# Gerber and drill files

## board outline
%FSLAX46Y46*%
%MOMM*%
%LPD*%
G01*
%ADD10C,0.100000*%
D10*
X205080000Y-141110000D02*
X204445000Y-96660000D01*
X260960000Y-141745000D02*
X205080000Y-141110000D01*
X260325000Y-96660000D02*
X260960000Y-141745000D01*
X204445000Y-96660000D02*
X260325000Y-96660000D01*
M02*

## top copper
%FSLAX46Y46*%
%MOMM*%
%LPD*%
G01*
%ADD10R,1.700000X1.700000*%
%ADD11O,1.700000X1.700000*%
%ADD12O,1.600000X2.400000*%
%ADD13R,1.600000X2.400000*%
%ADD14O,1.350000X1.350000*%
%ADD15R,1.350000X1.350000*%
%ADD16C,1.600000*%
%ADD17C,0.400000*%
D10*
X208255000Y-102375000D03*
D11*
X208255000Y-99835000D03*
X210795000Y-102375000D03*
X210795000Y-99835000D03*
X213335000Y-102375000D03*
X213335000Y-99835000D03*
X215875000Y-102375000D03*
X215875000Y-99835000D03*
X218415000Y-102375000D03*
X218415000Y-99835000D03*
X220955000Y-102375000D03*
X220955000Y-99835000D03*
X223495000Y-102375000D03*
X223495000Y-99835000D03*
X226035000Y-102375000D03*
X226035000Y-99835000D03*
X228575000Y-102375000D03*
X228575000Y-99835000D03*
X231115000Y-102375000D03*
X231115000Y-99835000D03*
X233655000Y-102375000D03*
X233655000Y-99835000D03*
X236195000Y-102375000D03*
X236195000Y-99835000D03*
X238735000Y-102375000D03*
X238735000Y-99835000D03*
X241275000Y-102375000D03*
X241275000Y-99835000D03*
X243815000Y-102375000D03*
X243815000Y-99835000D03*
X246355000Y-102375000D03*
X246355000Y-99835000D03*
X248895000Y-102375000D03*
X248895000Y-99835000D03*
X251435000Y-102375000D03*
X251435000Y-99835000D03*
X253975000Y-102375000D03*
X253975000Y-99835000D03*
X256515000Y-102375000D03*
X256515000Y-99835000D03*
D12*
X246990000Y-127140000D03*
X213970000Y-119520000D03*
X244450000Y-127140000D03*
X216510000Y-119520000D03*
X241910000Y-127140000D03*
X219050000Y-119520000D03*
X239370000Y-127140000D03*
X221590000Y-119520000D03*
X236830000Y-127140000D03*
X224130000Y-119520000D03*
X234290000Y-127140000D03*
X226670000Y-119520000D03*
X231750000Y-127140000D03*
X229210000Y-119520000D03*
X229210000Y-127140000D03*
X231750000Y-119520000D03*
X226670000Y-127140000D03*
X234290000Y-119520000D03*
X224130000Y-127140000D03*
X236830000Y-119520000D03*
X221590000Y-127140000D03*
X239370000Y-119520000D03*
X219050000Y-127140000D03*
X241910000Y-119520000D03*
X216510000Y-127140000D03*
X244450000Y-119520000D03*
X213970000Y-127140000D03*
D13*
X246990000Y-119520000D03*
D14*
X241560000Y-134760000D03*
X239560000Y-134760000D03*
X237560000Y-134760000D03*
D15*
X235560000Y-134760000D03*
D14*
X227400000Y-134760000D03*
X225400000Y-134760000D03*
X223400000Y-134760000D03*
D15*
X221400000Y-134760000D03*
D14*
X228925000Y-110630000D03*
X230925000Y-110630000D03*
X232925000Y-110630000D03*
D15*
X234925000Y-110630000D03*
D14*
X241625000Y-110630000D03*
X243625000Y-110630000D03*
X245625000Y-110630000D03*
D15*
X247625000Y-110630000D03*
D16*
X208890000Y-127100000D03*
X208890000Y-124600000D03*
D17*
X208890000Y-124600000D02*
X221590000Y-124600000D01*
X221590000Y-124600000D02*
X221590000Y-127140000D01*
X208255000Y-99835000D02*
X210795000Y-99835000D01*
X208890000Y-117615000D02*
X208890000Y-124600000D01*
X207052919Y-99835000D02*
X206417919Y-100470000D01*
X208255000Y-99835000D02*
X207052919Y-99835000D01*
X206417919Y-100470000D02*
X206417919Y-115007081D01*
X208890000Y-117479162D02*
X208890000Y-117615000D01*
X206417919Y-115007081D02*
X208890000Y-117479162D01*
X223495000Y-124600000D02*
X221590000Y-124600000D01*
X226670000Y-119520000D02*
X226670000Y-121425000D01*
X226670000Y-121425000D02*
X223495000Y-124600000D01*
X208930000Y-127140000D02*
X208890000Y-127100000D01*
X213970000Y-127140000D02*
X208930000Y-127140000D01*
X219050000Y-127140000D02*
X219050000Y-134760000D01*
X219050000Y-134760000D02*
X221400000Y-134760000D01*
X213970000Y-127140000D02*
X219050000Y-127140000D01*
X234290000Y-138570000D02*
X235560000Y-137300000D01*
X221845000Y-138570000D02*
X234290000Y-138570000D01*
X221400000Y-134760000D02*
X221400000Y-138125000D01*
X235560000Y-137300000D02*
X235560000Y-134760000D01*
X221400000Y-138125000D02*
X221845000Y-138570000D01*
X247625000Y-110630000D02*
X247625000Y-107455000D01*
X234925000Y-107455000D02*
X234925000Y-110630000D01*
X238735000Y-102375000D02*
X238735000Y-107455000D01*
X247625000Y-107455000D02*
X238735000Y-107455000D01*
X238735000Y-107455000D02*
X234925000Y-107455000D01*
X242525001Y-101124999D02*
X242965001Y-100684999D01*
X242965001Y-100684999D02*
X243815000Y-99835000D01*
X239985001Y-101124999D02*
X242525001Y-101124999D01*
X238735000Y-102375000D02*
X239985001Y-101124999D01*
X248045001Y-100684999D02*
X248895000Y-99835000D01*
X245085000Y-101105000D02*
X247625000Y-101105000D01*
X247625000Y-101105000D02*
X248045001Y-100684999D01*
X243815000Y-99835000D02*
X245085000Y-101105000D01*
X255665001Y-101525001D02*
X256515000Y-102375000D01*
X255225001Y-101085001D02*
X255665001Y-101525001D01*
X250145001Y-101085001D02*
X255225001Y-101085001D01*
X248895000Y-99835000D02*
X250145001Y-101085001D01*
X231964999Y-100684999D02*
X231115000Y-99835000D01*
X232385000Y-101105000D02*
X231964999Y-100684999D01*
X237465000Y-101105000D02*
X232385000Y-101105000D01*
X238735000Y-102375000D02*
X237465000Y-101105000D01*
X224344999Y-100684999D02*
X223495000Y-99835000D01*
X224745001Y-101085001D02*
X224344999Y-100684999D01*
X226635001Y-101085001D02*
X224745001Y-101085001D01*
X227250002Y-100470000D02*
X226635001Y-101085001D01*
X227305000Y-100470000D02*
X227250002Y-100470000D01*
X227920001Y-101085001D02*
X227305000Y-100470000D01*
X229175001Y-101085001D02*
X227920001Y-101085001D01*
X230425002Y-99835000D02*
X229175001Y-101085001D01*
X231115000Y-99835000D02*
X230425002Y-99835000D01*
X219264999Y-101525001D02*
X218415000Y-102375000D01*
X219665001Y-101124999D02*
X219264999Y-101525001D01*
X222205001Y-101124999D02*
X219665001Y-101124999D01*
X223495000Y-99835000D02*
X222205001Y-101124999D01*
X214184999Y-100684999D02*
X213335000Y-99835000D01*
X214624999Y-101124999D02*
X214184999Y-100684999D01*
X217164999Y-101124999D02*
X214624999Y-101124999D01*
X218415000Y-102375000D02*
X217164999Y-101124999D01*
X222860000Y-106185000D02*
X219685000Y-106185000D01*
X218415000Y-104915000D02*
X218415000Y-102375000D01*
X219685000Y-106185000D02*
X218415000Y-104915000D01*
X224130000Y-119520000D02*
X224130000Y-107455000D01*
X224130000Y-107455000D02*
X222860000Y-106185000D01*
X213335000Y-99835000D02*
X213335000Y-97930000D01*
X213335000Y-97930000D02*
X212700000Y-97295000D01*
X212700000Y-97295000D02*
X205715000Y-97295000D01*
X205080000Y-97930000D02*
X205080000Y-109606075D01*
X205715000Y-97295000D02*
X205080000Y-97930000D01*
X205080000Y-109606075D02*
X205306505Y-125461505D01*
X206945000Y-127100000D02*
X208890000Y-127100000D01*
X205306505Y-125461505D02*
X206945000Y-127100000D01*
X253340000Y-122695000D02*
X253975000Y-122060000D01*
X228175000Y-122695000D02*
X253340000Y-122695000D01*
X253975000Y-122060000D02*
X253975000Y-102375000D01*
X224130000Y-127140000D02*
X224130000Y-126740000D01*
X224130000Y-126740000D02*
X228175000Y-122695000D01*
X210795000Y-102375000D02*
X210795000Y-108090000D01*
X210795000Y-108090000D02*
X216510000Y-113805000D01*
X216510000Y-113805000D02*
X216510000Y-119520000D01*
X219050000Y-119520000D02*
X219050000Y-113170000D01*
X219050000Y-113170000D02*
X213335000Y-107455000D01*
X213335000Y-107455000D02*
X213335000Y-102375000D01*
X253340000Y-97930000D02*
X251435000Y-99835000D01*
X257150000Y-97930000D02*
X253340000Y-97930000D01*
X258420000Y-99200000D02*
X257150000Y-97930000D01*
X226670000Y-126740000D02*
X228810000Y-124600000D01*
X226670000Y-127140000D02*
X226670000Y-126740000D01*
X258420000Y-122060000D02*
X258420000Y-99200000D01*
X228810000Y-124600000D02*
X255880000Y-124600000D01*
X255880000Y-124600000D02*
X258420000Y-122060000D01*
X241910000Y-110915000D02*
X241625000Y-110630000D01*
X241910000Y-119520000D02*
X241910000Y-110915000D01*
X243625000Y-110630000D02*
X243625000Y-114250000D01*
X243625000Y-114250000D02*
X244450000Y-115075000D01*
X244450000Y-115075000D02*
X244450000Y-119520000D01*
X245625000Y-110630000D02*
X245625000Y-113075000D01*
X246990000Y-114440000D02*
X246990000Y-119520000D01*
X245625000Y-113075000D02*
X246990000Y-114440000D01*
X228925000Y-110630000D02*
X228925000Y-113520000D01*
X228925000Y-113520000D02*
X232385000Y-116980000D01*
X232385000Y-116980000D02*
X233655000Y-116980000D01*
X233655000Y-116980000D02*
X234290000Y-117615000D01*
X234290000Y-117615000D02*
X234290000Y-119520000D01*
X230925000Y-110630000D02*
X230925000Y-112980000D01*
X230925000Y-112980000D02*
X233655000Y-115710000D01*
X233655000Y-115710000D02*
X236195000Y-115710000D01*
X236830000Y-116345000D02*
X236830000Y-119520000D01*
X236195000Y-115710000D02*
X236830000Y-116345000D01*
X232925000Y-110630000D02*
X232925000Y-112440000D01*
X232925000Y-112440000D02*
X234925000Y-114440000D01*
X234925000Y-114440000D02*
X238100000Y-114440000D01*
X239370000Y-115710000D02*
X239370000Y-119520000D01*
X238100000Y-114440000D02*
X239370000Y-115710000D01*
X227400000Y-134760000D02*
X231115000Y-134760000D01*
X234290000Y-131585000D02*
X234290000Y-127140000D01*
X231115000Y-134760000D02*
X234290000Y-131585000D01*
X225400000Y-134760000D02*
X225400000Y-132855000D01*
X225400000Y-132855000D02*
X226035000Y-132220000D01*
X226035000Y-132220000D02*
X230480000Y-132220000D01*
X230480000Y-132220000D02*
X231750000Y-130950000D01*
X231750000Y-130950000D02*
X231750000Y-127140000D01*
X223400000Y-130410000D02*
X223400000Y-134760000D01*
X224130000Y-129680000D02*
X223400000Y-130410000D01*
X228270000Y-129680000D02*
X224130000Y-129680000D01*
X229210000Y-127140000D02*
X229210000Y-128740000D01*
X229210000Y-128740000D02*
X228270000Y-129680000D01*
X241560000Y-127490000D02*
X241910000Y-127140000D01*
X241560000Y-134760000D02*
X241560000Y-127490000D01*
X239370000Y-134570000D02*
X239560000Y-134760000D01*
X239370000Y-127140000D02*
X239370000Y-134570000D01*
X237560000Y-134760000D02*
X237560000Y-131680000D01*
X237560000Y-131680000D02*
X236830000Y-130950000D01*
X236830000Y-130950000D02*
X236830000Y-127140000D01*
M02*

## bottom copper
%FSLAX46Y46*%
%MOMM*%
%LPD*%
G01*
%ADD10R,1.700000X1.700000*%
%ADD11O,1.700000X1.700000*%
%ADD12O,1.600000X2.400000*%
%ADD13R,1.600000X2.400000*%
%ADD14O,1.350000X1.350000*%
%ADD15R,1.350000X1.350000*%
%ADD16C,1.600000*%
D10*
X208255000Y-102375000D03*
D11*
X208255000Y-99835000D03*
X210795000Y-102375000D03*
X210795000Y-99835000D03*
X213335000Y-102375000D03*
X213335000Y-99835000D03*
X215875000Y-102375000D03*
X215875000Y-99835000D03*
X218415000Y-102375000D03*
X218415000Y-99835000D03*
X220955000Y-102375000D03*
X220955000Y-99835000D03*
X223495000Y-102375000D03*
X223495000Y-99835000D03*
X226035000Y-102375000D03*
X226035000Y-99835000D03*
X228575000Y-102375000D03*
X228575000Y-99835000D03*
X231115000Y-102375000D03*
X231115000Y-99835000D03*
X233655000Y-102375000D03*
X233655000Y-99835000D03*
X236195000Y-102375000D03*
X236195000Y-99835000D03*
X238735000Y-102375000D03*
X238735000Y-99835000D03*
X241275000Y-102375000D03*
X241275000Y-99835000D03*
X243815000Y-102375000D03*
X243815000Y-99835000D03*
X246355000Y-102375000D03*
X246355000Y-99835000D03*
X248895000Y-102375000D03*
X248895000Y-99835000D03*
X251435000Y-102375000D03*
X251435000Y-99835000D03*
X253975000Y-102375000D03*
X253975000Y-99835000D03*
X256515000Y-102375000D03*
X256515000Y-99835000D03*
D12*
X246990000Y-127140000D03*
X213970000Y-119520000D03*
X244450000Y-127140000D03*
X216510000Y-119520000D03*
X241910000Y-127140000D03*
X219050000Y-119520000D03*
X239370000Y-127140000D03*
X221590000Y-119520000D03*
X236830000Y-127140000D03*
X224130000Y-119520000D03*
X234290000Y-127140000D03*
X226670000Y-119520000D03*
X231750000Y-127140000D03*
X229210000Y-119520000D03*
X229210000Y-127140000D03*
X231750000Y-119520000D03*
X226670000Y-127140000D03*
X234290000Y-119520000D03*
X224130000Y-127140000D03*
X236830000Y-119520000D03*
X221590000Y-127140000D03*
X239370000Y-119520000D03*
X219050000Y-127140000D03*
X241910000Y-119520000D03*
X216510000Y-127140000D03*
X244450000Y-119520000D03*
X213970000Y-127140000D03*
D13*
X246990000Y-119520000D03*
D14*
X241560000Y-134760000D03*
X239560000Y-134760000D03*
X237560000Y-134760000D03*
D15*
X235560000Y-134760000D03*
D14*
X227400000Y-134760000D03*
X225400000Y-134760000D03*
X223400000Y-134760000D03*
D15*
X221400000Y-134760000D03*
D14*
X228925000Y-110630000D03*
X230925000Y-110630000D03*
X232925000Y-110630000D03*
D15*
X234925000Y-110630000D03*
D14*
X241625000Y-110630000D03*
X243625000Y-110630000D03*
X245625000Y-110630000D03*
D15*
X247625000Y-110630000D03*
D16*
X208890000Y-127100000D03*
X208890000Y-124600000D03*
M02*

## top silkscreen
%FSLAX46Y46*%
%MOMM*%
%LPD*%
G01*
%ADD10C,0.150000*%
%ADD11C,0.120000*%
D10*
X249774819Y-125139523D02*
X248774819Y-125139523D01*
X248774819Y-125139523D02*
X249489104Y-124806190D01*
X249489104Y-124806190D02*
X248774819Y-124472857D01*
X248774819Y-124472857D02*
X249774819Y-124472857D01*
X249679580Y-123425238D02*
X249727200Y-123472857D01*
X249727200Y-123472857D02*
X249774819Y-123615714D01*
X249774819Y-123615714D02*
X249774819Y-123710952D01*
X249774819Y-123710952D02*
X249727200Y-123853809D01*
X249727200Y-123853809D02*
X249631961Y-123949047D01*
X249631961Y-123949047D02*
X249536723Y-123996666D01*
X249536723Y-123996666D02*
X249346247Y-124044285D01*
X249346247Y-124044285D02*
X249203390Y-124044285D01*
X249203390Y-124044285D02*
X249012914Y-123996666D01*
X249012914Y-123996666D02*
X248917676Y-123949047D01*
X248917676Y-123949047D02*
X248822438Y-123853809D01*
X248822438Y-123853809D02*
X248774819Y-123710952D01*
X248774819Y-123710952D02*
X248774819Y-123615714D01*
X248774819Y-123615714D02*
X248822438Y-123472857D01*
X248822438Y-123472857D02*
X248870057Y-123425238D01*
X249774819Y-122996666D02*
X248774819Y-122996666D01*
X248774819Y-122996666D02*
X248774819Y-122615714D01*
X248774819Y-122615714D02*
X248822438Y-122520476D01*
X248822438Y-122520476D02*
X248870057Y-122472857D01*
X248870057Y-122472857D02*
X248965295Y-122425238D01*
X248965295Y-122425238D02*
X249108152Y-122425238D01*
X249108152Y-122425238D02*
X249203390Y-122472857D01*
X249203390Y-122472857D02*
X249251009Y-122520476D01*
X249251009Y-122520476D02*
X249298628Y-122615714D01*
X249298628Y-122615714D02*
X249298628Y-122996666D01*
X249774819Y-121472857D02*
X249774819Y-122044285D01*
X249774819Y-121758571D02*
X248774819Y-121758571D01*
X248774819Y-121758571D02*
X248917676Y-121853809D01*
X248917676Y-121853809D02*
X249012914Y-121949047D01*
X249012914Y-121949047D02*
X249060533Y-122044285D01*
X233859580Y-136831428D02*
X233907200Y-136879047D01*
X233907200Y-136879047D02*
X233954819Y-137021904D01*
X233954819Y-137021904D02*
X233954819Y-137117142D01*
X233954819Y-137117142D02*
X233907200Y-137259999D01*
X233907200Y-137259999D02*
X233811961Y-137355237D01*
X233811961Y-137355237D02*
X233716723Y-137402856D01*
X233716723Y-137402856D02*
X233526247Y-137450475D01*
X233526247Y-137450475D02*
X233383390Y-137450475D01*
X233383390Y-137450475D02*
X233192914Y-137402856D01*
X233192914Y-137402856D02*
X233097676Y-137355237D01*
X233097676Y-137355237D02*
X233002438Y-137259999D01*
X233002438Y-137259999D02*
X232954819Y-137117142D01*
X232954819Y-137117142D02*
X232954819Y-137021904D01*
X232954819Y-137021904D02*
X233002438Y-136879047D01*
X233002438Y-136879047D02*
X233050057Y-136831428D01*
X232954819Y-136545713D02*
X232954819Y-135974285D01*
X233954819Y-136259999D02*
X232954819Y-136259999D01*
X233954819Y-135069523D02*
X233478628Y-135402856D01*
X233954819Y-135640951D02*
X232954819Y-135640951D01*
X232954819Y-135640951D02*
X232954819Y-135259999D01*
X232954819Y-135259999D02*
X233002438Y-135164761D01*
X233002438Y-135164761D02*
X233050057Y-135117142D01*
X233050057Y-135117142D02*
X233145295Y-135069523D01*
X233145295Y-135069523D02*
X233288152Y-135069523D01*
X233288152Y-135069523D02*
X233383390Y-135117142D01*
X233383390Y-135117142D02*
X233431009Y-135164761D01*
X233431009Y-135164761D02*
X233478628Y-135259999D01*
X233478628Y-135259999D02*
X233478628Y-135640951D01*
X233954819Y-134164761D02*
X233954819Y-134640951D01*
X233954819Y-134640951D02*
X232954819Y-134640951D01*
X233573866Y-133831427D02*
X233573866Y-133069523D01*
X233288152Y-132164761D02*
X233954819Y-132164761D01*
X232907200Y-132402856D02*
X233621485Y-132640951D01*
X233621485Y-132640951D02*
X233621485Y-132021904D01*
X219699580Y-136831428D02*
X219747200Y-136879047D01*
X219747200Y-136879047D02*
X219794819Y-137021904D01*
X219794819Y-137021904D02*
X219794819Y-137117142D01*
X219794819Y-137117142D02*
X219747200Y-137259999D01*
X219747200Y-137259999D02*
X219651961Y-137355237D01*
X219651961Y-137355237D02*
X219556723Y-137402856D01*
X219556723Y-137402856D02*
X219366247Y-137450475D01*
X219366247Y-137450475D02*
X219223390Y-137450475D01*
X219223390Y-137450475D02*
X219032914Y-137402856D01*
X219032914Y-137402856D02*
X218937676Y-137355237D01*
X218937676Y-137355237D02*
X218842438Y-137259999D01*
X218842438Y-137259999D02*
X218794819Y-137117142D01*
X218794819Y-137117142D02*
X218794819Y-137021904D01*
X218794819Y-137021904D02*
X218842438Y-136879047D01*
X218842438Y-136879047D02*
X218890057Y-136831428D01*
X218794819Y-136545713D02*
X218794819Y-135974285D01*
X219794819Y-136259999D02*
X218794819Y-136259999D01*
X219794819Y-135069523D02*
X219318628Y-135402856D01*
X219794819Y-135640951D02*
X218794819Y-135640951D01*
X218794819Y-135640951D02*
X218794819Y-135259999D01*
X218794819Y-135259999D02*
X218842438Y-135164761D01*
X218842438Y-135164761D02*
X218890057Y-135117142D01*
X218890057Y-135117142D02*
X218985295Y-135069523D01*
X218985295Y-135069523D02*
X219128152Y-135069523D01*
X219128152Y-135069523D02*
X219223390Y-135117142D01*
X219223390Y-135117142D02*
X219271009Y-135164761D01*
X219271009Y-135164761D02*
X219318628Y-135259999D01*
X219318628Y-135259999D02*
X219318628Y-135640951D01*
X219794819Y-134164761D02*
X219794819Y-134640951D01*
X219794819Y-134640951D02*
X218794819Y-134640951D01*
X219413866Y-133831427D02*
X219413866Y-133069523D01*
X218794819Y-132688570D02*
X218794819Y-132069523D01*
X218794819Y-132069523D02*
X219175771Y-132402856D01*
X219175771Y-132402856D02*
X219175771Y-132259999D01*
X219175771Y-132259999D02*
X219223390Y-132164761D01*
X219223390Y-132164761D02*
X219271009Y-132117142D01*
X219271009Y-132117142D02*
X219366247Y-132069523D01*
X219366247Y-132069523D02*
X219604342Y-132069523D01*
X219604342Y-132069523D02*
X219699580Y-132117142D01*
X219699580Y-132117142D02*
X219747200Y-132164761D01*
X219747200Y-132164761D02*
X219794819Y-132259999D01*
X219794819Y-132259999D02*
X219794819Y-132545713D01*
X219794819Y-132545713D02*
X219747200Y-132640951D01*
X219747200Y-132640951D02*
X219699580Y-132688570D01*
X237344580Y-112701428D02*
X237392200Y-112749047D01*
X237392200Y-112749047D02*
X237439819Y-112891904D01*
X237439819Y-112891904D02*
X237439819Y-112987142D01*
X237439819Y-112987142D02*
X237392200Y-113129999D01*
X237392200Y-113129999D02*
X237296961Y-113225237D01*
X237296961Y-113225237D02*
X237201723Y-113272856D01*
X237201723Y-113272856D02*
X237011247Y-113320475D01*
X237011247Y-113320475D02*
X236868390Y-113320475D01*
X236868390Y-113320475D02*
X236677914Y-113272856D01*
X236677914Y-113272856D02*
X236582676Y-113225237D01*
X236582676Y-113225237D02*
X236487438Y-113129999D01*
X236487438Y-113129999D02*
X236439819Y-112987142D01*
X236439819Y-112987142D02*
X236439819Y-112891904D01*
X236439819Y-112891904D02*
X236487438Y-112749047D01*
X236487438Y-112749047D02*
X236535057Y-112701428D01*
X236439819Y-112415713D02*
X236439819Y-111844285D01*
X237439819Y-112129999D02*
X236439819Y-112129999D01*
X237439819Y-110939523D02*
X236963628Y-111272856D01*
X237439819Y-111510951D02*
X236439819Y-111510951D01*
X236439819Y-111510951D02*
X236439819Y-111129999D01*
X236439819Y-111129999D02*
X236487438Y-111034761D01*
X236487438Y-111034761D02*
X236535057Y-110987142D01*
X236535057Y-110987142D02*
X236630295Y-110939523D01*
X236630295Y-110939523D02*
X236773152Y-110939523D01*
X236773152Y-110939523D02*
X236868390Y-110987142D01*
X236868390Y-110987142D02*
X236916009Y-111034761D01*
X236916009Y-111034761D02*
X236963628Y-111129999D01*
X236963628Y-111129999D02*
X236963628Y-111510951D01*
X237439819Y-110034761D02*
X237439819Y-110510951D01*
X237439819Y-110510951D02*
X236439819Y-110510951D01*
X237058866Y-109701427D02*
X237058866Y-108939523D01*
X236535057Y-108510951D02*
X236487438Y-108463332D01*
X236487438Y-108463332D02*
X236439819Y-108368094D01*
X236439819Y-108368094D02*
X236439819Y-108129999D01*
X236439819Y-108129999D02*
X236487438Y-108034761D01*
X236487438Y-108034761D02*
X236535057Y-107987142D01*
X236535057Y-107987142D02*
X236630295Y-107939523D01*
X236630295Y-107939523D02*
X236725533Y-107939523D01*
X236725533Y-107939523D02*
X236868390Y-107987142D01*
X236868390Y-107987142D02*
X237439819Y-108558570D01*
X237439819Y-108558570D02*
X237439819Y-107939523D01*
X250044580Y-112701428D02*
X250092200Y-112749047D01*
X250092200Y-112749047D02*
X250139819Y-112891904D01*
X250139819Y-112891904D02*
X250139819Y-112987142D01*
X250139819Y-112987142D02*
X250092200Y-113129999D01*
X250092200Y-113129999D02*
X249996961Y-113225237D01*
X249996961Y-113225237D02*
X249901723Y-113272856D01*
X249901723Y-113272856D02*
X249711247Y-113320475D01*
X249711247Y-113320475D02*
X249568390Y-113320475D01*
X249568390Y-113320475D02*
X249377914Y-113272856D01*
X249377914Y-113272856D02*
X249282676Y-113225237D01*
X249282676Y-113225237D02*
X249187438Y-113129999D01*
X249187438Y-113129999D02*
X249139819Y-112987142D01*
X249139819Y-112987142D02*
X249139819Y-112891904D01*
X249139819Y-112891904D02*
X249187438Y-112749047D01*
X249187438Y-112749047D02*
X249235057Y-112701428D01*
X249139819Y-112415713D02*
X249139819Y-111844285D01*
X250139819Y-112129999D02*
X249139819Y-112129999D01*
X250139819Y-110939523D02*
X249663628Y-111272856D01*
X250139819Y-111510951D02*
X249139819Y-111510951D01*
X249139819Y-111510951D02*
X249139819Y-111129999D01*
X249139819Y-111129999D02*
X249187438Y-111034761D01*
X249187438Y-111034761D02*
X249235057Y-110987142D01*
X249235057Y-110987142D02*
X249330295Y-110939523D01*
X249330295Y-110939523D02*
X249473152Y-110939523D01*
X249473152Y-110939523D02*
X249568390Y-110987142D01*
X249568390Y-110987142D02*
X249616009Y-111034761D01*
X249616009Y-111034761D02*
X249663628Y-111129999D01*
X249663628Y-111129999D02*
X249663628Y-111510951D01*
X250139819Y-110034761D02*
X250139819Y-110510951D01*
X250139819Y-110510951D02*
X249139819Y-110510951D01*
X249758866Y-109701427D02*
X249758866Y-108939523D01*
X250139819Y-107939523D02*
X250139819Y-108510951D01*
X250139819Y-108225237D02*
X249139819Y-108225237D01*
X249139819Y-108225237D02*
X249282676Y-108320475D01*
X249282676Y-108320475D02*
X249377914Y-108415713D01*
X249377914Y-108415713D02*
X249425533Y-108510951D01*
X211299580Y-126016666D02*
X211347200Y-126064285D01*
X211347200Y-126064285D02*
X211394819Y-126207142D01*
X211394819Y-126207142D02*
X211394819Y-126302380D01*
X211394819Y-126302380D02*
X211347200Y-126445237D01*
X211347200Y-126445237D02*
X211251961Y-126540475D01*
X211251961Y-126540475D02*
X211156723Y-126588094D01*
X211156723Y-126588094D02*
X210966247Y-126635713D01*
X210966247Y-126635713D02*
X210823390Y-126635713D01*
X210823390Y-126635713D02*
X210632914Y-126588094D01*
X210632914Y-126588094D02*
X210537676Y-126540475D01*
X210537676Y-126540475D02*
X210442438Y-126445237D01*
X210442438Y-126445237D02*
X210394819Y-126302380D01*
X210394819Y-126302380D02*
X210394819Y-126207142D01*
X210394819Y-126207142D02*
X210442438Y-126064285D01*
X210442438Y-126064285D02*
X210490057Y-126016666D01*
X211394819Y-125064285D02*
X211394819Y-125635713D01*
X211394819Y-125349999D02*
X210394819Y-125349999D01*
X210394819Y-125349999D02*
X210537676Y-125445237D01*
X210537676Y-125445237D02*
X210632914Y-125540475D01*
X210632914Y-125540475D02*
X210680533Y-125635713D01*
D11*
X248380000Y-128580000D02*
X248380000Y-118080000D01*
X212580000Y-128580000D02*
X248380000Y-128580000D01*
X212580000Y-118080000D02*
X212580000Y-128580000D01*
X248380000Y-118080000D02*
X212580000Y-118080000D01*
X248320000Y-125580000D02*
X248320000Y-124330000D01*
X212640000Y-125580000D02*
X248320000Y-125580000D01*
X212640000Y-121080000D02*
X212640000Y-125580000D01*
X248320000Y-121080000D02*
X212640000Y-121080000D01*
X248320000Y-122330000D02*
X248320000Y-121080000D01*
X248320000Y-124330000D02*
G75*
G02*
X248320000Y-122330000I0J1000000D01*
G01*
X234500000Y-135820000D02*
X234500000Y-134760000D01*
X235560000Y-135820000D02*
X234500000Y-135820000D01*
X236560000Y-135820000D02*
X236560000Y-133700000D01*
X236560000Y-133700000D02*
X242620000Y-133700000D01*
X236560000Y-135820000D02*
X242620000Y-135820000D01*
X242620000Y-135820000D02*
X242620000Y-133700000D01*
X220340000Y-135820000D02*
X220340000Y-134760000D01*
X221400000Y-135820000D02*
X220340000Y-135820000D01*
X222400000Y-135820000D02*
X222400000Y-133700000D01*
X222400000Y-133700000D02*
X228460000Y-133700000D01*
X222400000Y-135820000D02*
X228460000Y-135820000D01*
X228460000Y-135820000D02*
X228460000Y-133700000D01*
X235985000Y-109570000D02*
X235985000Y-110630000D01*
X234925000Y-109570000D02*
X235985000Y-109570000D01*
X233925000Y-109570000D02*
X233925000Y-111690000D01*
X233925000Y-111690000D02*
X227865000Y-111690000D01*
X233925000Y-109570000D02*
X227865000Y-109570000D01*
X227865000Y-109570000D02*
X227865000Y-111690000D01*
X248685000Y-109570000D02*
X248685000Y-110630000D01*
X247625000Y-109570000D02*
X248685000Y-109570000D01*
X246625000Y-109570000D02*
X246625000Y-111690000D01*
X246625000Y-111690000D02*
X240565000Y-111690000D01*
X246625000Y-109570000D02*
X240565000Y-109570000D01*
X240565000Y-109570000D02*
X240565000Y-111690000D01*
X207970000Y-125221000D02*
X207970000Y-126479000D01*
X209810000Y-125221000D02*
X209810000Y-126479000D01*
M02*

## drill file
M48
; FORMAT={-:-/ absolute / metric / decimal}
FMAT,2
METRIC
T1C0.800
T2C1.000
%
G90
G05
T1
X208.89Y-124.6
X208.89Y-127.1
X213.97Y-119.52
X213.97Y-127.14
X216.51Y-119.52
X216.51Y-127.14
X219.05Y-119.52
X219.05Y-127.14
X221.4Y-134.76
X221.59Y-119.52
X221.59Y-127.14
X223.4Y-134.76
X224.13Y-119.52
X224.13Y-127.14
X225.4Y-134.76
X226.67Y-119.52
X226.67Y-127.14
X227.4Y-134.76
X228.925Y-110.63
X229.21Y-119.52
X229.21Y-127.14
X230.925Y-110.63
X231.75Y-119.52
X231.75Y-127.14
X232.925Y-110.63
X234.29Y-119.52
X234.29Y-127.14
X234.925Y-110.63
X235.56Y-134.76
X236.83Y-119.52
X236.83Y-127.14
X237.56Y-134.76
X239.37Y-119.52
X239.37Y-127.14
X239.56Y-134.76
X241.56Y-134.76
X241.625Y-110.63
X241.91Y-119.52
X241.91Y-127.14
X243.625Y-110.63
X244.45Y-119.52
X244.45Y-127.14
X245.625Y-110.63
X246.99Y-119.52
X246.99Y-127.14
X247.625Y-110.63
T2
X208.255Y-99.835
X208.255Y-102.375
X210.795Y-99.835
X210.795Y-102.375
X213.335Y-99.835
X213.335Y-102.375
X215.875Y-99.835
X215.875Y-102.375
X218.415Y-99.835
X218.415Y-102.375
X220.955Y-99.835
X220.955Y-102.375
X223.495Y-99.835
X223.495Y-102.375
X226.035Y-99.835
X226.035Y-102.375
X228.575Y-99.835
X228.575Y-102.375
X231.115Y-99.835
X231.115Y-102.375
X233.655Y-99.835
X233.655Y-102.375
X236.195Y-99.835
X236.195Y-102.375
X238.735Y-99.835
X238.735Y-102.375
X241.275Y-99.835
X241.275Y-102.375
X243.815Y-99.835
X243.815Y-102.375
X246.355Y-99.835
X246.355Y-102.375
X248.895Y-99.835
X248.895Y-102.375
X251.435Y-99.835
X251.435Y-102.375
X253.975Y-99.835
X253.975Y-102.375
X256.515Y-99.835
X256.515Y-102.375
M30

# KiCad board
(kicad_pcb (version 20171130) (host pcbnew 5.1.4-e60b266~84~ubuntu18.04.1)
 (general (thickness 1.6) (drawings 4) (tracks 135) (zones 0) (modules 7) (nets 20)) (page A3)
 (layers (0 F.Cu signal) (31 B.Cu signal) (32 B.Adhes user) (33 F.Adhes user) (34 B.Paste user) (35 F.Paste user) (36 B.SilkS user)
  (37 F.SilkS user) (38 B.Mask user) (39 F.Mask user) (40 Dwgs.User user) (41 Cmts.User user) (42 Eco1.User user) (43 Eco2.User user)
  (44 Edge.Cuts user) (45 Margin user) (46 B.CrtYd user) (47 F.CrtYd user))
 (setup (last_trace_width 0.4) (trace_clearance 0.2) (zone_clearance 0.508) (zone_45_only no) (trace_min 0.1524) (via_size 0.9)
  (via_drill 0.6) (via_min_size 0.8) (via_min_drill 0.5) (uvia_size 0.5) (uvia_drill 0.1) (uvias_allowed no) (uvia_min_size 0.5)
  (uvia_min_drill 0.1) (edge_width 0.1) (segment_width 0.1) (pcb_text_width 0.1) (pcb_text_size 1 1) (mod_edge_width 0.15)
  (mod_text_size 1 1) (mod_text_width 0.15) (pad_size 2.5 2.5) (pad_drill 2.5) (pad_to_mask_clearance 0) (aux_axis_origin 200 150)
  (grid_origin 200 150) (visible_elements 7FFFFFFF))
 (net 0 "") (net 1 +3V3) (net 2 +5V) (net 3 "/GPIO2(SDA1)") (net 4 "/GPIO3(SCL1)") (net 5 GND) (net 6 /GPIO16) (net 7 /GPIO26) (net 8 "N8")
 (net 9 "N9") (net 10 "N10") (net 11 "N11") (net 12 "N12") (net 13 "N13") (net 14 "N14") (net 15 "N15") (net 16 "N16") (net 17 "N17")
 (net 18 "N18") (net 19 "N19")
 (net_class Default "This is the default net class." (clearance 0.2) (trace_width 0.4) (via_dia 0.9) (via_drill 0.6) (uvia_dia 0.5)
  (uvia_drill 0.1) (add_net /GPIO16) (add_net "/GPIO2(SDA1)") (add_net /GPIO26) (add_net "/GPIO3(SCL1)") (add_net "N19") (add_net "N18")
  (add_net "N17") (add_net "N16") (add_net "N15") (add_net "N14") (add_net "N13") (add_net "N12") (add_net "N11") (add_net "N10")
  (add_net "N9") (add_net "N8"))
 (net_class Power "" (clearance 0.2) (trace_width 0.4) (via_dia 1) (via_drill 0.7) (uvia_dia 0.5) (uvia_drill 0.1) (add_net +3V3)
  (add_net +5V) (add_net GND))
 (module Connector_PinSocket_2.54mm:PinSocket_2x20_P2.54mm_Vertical (layer B.Cu) (at 208.255 102.375 270)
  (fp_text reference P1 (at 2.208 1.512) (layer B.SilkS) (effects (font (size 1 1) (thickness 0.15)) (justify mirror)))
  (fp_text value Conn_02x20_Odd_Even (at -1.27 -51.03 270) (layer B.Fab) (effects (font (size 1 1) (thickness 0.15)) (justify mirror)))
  (pad 1 thru_hole rect (at 0 0 270) (size 1.7 1.7) (drill 1) (layers *.Cu *.Mask) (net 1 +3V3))
  (pad 2 thru_hole oval (at -2.54 0 270) (size 1.7 1.7) (drill 1) (layers *.Cu *.Mask) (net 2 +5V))
  (pad 3 thru_hole oval (at 0 -2.54 270) (size 1.7 1.7) (drill 1) (layers *.Cu *.Mask) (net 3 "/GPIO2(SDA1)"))
  (pad 4 thru_hole oval (at -2.54 -2.54 270) (size 1.7 1.7) (drill 1) (layers *.Cu *.Mask) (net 2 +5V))
  (pad 5 thru_hole oval (at 0 -5.08 270) (size 1.7 1.7) (drill 1) (layers *.Cu *.Mask) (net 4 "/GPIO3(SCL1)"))
  (pad 6 thru_hole oval (at -2.54 -5.08 270) (size 1.7 1.7) (drill 1) (layers *.Cu *.Mask) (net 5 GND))
  (pad 7 thru_hole oval (at 0 -7.62 270) (size 1.7 1.7) (drill 1) (layers *.Cu *.Mask))
  (pad 8 thru_hole oval (at -2.54 -7.62 270) (size 1.7 1.7) (drill 1) (layers *.Cu *.Mask))
  (pad 9 thru_hole oval (at 0 -10.16 270) (size 1.7 1.7) (drill 1) (layers *.Cu *.Mask) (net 5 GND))
  (pad 10 thru_hole oval (at -2.54 -10.16 270) (size 1.7 1.7) (drill 1) (layers *.Cu *.Mask))
  (pad 11 thru_hole oval (at 0 -12.7 270) (size 1.7 1.7) (drill 1) (layers *.Cu *.Mask))
  (pad 12 thru_hole oval (at -2.54 -12.7 270) (size 1.7 1.7) (drill 1) (layers *.Cu *.Mask))
  (pad 13 thru_hole oval (at 0 -15.24 270) (size 1.7 1.7) (drill 1) (layers *.Cu *.Mask))
  (pad 14 thru_hole oval (at -2.54 -15.24 270) (size 1.7 1.7) (drill 1) (layers *.Cu *.Mask) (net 5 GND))
  (pad 15 thru_hole oval (at 0 -17.78 270) (size 1.7 1.7) (drill 1) (layers *.Cu *.Mask))
  (pad 16 thru_hole oval (at -2.54 -17.78 270) (size 1.7 1.7) (drill 1) (layers *.Cu *.Mask))
  (pad 17 thru_hole oval (at 0 -20.32 270) (size 1.7 1.7) (drill 1) (layers *.Cu *.Mask) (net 1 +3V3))
  (pad 18 thru_hole oval (at -2.54 -20.32 270) (size 1.7 1.7) (drill 1) (layers *.Cu *.Mask))
  (pad 19 thru_hole oval (at 0 -22.86 270) (size 1.7 1.7) (drill 1) (layers *.Cu *.Mask))
  (pad 20 thru_hole oval (at -2.54 -22.86 270) (size 1.7 1.7) (drill 1) (layers *.Cu *.Mask) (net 5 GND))
  (pad 21 thru_hole oval (at 0 -25.4 270) (size 1.7 1.7) (drill 1) (layers *.Cu *.Mask))
  (pad 22 thru_hole oval (at -2.54 -25.4 270) (size 1.7 1.7) (drill 1) (layers *.Cu *.Mask))
  (pad 23 thru_hole oval (at 0 -27.94 270) (size 1.7 1.7) (drill 1) (layers *.Cu *.Mask))
  (pad 24 thru_hole oval (at -2.54 -27.94 270) (size 1.7 1.7) (drill 1) (layers *.Cu *.Mask))
  (pad 25 thru_hole oval (at 0 -30.48 270) (size 1.7 1.7) (drill 1) (layers *.Cu *.Mask) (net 5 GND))
  (pad 26 thru_hole oval (at -2.54 -30.48 270) (size 1.7 1.7) (drill 1) (layers *.Cu *.Mask))
  (pad 27 thru_hole oval (at 0 -33.02 270) (size 1.7 1.7) (drill 1) (layers *.Cu *.Mask))
  (pad 28 thru_hole oval (at -2.54 -33.02 270) (size 1.7 1.7) (drill 1) (layers *.Cu *.Mask))
  (pad 29 thru_hole oval (at 0 -35.56 270) (size 1.7 1.7) (drill 1) (layers *.Cu *.Mask))
  (pad 30 thru_hole oval (at -2.54 -35.56 270) (size 1.7 1.7) (drill 1) (layers *.Cu *.Mask) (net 5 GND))
  (pad 31 thru_hole oval (at 0 -38.1 270) (size 1.7 1.7) (drill 1) (layers *.Cu *.Mask))
  (pad 32 thru_hole oval (at -2.54 -38.1 270) (size 1.7 1.7) (drill 1) (layers *.Cu *.Mask))
  (pad 33 thru_hole oval (at 0 -40.64 270) (size 1.7 1.7) (drill 1) (layers *.Cu *.Mask))
  (pad 34 thru_hole oval (at -2.54 -40.64 270) (size 1.7 1.7) (drill 1) (layers *.Cu *.Mask) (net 5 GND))
  (pad 35 thru_hole oval (at 0 -43.18 270) (size 1.7 1.7) (drill 1) (layers *.Cu *.Mask))
  (pad 36 thru_hole oval (at -2.54 -43.18 270) (size 1.7 1.7) (drill 1) (layers *.Cu *.Mask) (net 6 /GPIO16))
  (pad 37 thru_hole oval (at 0 -45.72 270) (size 1.7 1.7) (drill 1) (layers *.Cu *.Mask) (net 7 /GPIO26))
  (pad 38 thru_hole oval (at -2.54 -45.72 270) (size 1.7 1.7) (drill 1) (layers *.Cu *.Mask))
  (pad 39 thru_hole oval (at 0 -48.26 270) (size 1.7 1.7) (drill 1) (layers *.Cu *.Mask) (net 5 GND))
  (pad 40 thru_hole oval (at -2.54 -48.26 270) (size 1.7 1.7) (drill 1) (layers *.Cu *.Mask)))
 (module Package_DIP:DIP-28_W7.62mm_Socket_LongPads (layer F.Cu) (at 246.99 119.52 270)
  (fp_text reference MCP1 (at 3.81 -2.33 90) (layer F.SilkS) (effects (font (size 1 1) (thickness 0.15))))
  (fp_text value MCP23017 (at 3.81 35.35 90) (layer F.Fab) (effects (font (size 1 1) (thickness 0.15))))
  (fp_line (start 9.06 -1.39) (end -1.44 -1.39) (layer F.SilkS) (width 0.12))
  (fp_line (start 9.06 34.41) (end 9.06 -1.39) (layer F.SilkS) (width 0.12))
  (fp_line (start -1.44 34.41) (end 9.06 34.41) (layer F.SilkS) (width 0.12))
  (fp_line (start -1.44 -1.39) (end -1.44 34.41) (layer F.SilkS) (width 0.12))
  (fp_line (start 6.06 -1.33) (end 4.81 -1.33) (layer F.SilkS) (width 0.12))
  (fp_line (start 6.06 34.35) (end 6.06 -1.33) (layer F.SilkS) (width 0.12))
  (fp_line (start 1.56 34.35) (end 6.06 34.35) (layer F.SilkS) (width 0.12))
  (fp_line (start 1.56 -1.33) (end 1.56 34.35) (layer F.SilkS) (width 0.12))
  (fp_line (start 2.81 -1.33) (end 1.56 -1.33) (layer F.SilkS) (width 0.12))
  (fp_arc (start 3.81 -1.33) (end 2.81 -1.33) (angle -180) (layer F.SilkS) (width 0.12))
  (pad 28 thru_hole oval (at 7.62 0 270) (size 2.4 1.6) (drill 0.8) (layers *.Cu *.Mask))
  (pad 14 thru_hole oval (at 0 33.02 270) (size 2.4 1.6) (drill 0.8) (layers *.Cu *.Mask))
  (pad 27 thru_hole oval (at 7.62 2.54 270) (size 2.4 1.6) (drill 0.8) (layers *.Cu *.Mask))
  (pad 13 thru_hole oval (at 0 30.48 270) (size 2.4 1.6) (drill 0.8) (layers *.Cu *.Mask) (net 3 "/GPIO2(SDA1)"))
  (pad 26 thru_hole oval (at 7.62 5.08 270) (size 2.4 1.6) (drill 0.8) (layers *.Cu *.Mask) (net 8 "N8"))
  (pad 12 thru_hole oval (at 0 27.94 270) (size 2.4 1.6) (drill 0.8) (layers *.Cu *.Mask) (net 4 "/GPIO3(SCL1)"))
  (pad 25 thru_hole oval (at 7.62 7.62 270) (size 2.4 1.6) (drill 0.8) (layers *.Cu *.Mask) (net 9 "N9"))
  (pad 11 thru_hole oval (at 0 25.4 270) (size 2.4 1.6) (drill 0.8) (layers *.Cu *.Mask))
  (pad 24 thru_hole oval (at 7.62 10.16 270) (size 2.4 1.6) (drill 0.8) (layers *.Cu *.Mask) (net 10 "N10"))
  (pad 10 thru_hole oval (at 0 22.86 270) (size 2.4 1.6) (drill 0.8) (layers *.Cu *.Mask) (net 5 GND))
  (pad 23 thru_hole oval (at 7.62 12.7 270) (size 2.4 1.6) (drill 0.8) (layers *.Cu *.Mask) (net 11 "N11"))
  (pad 9 thru_hole oval (at 0 20.32 270) (size 2.4 1.6) (drill 0.8) (layers *.Cu *.Mask) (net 2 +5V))
  (pad 22 thru_hole oval (at 7.62 15.24 270) (size 2.4 1.6) (drill 0.8) (layers *.Cu *.Mask) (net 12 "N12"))
  (pad 8 thru_hole oval (at 0 17.78 270) (size 2.4 1.6) (drill 0.8) (layers *.Cu *.Mask))
  (pad 21 thru_hole oval (at 7.62 17.78 270) (size 2.4 1.6) (drill 0.8) (layers *.Cu *.Mask) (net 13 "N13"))
  (pad 7 thru_hole oval (at 0 15.24 270) (size 2.4 1.6) (drill 0.8) (layers *.Cu *.Mask))
  (pad 20 thru_hole oval (at 7.62 20.32 270) (size 2.4 1.6) (drill 0.8) (layers *.Cu *.Mask) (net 6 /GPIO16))
  (pad 6 thru_hole oval (at 0 12.7 270) (size 2.4 1.6) (drill 0.8) (layers *.Cu *.Mask) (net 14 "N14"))
  (pad 19 thru_hole oval (at 7.62 22.86 270) (size 2.4 1.6) (drill 0.8) (layers *.Cu *.Mask) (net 7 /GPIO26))
  (pad 5 thru_hole oval (at 0 10.16 270) (size 2.4 1.6) (drill 0.8) (layers *.Cu *.Mask) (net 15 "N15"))
  (pad 18 thru_hole oval (at 7.62 25.4 270) (size 2.4 1.6) (drill 0.8) (layers *.Cu *.Mask) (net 2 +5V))
  (pad 4 thru_hole oval (at 0 7.62 270) (size 2.4 1.6) (drill 0.8) (layers *.Cu *.Mask) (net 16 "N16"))
  (pad 17 thru_hole oval (at 7.62 27.94 270) (size 2.4 1.6) (drill 0.8) (layers *.Cu *.Mask) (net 5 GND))
  (pad 3 thru_hole oval (at 0 5.08 270) (size 2.4 1.6) (drill 0.8) (layers *.Cu *.Mask) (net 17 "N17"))
  (pad 16 thru_hole oval (at 7.62 30.48 270) (size 2.4 1.6) (drill 0.8) (layers *.Cu *.Mask) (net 5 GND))
  (pad 2 thru_hole oval (at 0 2.54 270) (size 2.4 1.6) (drill 0.8) (layers *.Cu *.Mask) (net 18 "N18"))
  (pad 15 thru_hole oval (at 7.62 33.02 270) (size 2.4 1.6) (drill 0.8) (layers *.Cu *.Mask) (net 5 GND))
  (pad 1 thru_hole rect (at 0 0 270) (size 2.4 1.6) (drill 0.8) (layers *.Cu *.Mask) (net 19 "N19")))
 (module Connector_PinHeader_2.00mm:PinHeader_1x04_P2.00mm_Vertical (layer F.Cu) (at 235.56 134.76 90)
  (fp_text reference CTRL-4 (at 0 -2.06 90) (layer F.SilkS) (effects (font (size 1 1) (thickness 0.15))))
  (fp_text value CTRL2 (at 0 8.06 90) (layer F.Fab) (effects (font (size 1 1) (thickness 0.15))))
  (fp_line (start -1.06 -1.06) (end 0 -1.06) (layer F.SilkS) (width 0.12))
  (fp_line (start -1.06 0) (end -1.06 -1.06) (layer F.SilkS) (width 0.12))
  (fp_line (start -1.06 1) (end 1.06 1) (layer F.SilkS) (width 0.12))
  (fp_line (start 1.06 1) (end 1.06 7.06) (layer F.SilkS) (width 0.12))
  (fp_line (start -1.06 1) (end -1.06 7.06) (layer F.SilkS) (width 0.12))
  (fp_line (start -1.06 7.06) (end 1.06 7.06) (layer F.SilkS) (width 0.12))
  (pad 4 thru_hole oval (at 0 6 90) (size 1.35 1.35) (drill 0.8) (layers *.Cu *.Mask) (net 8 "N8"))
  (pad 3 thru_hole oval (at 0 4 90) (size 1.35 1.35) (drill 0.8) (layers *.Cu *.Mask) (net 9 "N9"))
  (pad 2 thru_hole oval (at 0 2 90) (size 1.35 1.35) (drill 0.8) (layers *.Cu *.Mask) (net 10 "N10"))
  (pad 1 thru_hole rect (at 0 0 90) (size 1.35 1.35) (drill 0.8) (layers *.Cu *.Mask) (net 5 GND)))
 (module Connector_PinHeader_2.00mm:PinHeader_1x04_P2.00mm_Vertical (layer F.Cu) (at 221.4 134.76 90)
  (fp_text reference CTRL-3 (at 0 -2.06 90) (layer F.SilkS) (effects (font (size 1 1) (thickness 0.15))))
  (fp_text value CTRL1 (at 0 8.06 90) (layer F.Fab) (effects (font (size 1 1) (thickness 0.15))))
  (fp_line (start -1.06 -1.06) (end 0 -1.06) (layer F.SilkS) (width 0.12))
  (fp_line (start -1.06 0) (end -1.06 -1.06) (layer F.SilkS) (width 0.12))
  (fp_line (start -1.06 1) (end 1.06 1) (layer F.SilkS) (width 0.12))
  (fp_line (start 1.06 1) (end 1.06 7.06) (layer F.SilkS) (width 0.12))
  (fp_line (start -1.06 1) (end -1.06 7.06) (layer F.SilkS) (width 0.12))
  (fp_line (start -1.06 7.06) (end 1.06 7.06) (layer F.SilkS) (width 0.12))
  (pad 4 thru_hole oval (at 0 6 90) (size 1.35 1.35) (drill 0.8) (layers *.Cu *.Mask) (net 11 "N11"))
  (pad 3 thru_hole oval (at 0 4 90) (size 1.35 1.35) (drill 0.8) (layers *.Cu *.Mask) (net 12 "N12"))
  (pad 2 thru_hole oval (at 0 2 90) (size 1.35 1.35) (drill 0.8) (layers *.Cu *.Mask) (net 13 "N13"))
  (pad 1 thru_hole rect (at 0 0 90) (size 1.35 1.35) (drill 0.8) (layers *.Cu *.Mask) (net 5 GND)))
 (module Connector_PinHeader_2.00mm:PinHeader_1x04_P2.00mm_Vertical (layer F.Cu) (at 234.925 110.63 270)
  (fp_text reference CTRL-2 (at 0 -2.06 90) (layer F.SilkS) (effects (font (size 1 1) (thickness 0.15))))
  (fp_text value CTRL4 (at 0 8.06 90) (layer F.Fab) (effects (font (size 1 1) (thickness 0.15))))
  (fp_line (start -1.06 -1.06) (end 0 -1.06) (layer F.SilkS) (width 0.12))
  (fp_line (start -1.06 0) (end -1.06 -1.06) (layer F.SilkS) (width 0.12))
  (fp_line (start -1.06 1) (end 1.06 1) (layer F.SilkS) (width 0.12))
  (fp_line (start 1.06 1) (end 1.06 7.06) (layer F.SilkS) (width 0.12))
  (fp_line (start -1.06 1) (end -1.06 7.06) (layer F.SilkS) (width 0.12))
  (fp_line (start -1.06 7.06) (end 1.06 7.06) (layer F.SilkS) (width 0.12))
  (pad 4 thru_hole oval (at 0 6 270) (size 1.35 1.35) (drill 0.8) (layers *.Cu *.Mask) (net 14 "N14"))
  (pad 3 thru_hole oval (at 0 4 270) (size 1.35 1.35) (drill 0.8) (layers *.Cu *.Mask) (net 15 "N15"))
  (pad 2 thru_hole oval (at 0 2 270) (size 1.35 1.35) (drill 0.8) (layers *.Cu *.Mask) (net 16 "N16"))
  (pad 1 thru_hole rect (at 0 0 270) (size 1.35 1.35) (drill 0.8) (layers *.Cu *.Mask) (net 5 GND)))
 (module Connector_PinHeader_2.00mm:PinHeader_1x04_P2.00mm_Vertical (layer F.Cu) (at 247.625 110.63 270)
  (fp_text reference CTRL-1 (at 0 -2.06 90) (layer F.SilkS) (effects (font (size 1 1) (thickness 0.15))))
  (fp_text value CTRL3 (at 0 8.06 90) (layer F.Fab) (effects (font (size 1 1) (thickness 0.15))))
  (fp_line (start -1.06 -1.06) (end 0 -1.06) (layer F.SilkS) (width 0.12))
  (fp_line (start -1.06 0) (end -1.06 -1.06) (layer F.SilkS) (width 0.12))
  (fp_line (start -1.06 1) (end 1.06 1) (layer F.SilkS) (width 0.12))
  (fp_line (start 1.06 1) (end 1.06 7.06) (layer F.SilkS) (width 0.12))
  (fp_line (start -1.06 1) (end -1.06 7.06) (layer F.SilkS) (width 0.12))
  (fp_line (start -1.06 7.06) (end 1.06 7.06) (layer F.SilkS) (width 0.12))
  (pad 4 thru_hole oval (at 0 6 270) (size 1.35 1.35) (drill 0.8) (layers *.Cu *.Mask) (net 17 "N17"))
  (pad 3 thru_hole oval (at 0 4 270) (size 1.35 1.35) (drill 0.8) (layers *.Cu *.Mask) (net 18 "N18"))
  (pad 2 thru_hole oval (at 0 2 270) (size 1.35 1.35) (drill 0.8) (layers *.Cu *.Mask) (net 19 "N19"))
  (pad 1 thru_hole rect (at 0 0 270) (size 1.35 1.35) (drill 0.8) (layers *.Cu *.Mask) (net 5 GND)))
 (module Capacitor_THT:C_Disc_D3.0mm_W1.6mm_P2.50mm (layer F.Cu) (at 208.89 124.6 270)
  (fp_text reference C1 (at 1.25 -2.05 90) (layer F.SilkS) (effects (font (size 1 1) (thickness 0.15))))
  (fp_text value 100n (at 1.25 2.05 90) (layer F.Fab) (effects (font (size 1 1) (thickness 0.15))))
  (fp_line (start 0.621 0.92) (end 1.879 0.92) (layer F.SilkS) (width 0.12))
  (fp_line (start 0.621 -0.92) (end 1.879 -0.92) (layer F.SilkS) (width 0.12))
  (pad 2 thru_hole circle (at 2.5 0 270) (size 1.6 1.6) (drill 0.8) (layers *.Cu *.Mask) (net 5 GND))
  (pad 1 thru_hole circle (at 0 0 270) (size 1.6 1.6) (drill 0.8) (layers *.Cu *.Mask) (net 2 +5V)))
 (gr_line (start 205.08 141.11) (end 204.445 96.66) (layer Edge.Cuts) (width 0.1))
 (gr_line (start 260.96 141.745) (end 205.08 141.11) (layer Edge.Cuts) (width 0.1))
 (gr_line (start 260.325 96.66) (end 260.96 141.745) (layer Edge.Cuts) (width 0.1))
 (gr_line (start 204.445 96.66) (end 260.325 96.66) (layer Edge.Cuts) (width 0.1))
 (segment (start 208.89 124.6) (end 221.59 124.6) (width 0.4) (layer F.Cu) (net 2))
 (segment (start 221.59 124.6) (end 221.59 127.14) (width 0.4) (layer F.Cu) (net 2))
 (segment (start 208.255 99.835) (end 210.795 99.835) (width 0.4) (layer F.Cu) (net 2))
 (segment (start 208.89 117.615) (end 208.89 124.6) (width 0.4) (layer F.Cu) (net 2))
 (segment (start 207.052919 99.835) (end 206.417919 100.47) (width 0.4) (layer F.Cu) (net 2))
 (segment (start 208.255 99.835) (end 207.052919 99.835) (width 0.4) (layer F.Cu) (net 2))
 (segment (start 206.417919 100.47) (end 206.417919 115.007081) (width 0.4) (layer F.Cu) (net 2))
 (segment (start 208.89 117.479162) (end 208.89 117.615) (width 0.4) (layer F.Cu) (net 2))
 (segment (start 206.417919 115.007081) (end 208.89 117.479162) (width 0.4) (layer F.Cu) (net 2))
 (segment (start 223.495 124.6) (end 221.59 124.6) (width 0.4) (layer F.Cu) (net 2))
 (segment (start 226.67 119.52) (end 226.67 121.425) (width 0.4) (layer F.Cu) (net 2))
 (segment (start 226.67 121.425) (end 223.495 124.6) (width 0.4) (layer F.Cu) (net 2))
 (segment (start 208.93 127.14) (end 208.89 127.1) (width 0.4) (layer F.Cu) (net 5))
 (segment (start 213.97 127.14) (end 208.93 127.14) (width 0.4) (layer F.Cu) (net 5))
 (segment (start 219.05 127.14) (end 219.05 134.76) (width 0.4) (layer F.Cu) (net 5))
 (segment (start 219.05 134.76) (end 221.4 134.76) (width 0.4) (layer F.Cu) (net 5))
 (segment (start 213.97 127.14) (end 219.05 127.14) (width 0.4) (layer F.Cu) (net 5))
 (segment (start 234.29 138.57) (end 235.56 137.3) (width 0.4) (layer F.Cu) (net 5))
 (segment (start 221.845 138.57) (end 234.29 138.57) (width 0.4) (layer F.Cu) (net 5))
 (segment (start 221.4 134.76) (end 221.4 138.125) (width 0.4) (layer F.Cu) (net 5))
 (segment (start 235.56 137.3) (end 235.56 134.76) (width 0.4) (layer F.Cu) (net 5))
 (segment (start 221.4 138.125) (end 221.845 138.57) (width 0.4) (layer F.Cu) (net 5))
 (segment (start 247.625 110.63) (end 247.625 107.455) (width 0.4) (layer F.Cu) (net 5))
 (segment (start 234.925 107.455) (end 234.925 110.63) (width 0.4) (layer F.Cu) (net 5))
 (segment (start 238.735 102.375) (end 238.735 107.455) (width 0.4) (layer F.Cu) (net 5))
 (segment (start 247.625 107.455) (end 238.735 107.455) (width 0.4) (layer F.Cu) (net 5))
 (segment (start 238.735 107.455) (end 234.925 107.455) (width 0.4) (layer F.Cu) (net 5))
 (segment (start 242.525001 101.124999) (end 242.965001 100.684999) (width 0.4) (layer F.Cu) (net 5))
 (segment (start 242.965001 100.684999) (end 243.815 99.835) (width 0.4) (layer F.Cu) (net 5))
 (segment (start 239.985001 101.124999) (end 242.525001 101.124999) (width 0.4) (layer F.Cu) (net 5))
 (segment (start 238.735 102.375) (end 239.985001 101.124999) (width 0.4) (layer F.Cu) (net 5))
 (segment (start 248.045001 100.684999) (end 248.895 99.835) (width 0.4) (layer F.Cu) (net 5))
 (segment (start 245.085 101.105) (end 247.625 101.105) (width 0.4) (layer F.Cu) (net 5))
 (segment (start 247.625 101.105) (end 248.045001 100.684999) (width 0.4) (layer F.Cu) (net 5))
 (segment (start 243.815 99.835) (end 245.085 101.105) (width 0.4) (layer F.Cu) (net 5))
 (segment (start 255.665001 101.525001) (end 256.515 102.375) (width 0.4) (layer F.Cu) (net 5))
 (segment (start 255.225001 101.085001) (end 255.665001 101.525001) (width 0.4) (layer F.Cu) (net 5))
 (segment (start 250.145001 101.085001) (end 255.225001 101.085001) (width 0.4) (layer F.Cu) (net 5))
 (segment (start 248.895 99.835) (end 250.145001 101.085001) (width 0.4) (layer F.Cu) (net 5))
 (segment (start 231.964999 100.684999) (end 231.115 99.835) (width 0.4) (layer F.Cu) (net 5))
 (segment (start 232.385 101.105) (end 231.964999 100.684999) (width 0.4) (layer F.Cu) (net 5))
 (segment (start 237.465 101.105) (end 232.385 101.105) (width 0.4) (layer F.Cu) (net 5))
 (segment (start 238.735 102.375) (end 237.465 101.105) (width 0.4) (layer F.Cu) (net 5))
 (segment (start 224.344999 100.684999) (end 223.495 99.835) (width 0.4) (layer F.Cu) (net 5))
 (segment (start 224.745001 101.085001) (end 224.344999 100.684999) (width 0.4) (layer F.Cu) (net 5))
 (segment (start 226.635001 101.085001) (end 224.745001 101.085001) (width 0.4) (layer F.Cu) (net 5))
 (segment (start 227.250002 100.47) (end 226.635001 101.085001) (width 0.4) (layer F.Cu) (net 5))
 (segment (start 227.305 100.47) (end 227.250002 100.47) (width 0.4) (layer F.Cu) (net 5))
 (segment (start 227.920001 101.085001) (end 227.305 100.47) (width 0.4) (layer F.Cu) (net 5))
 (segment (start 229.175001 101.085001) (end 227.920001 101.085001) (width 0.4) (layer F.Cu) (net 5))
 (segment (start 230.425002 99.835) (end 229.175001 101.085001) (width 0.4) (layer F.Cu) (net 5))
 (segment (start 231.115 99.835) (end 230.425002 99.835) (width 0.4) (layer F.Cu) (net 5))
 (segment (start 219.264999 101.525001) (end 218.415 102.375) (width 0.4) (layer F.Cu) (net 5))
 (segment (start 219.665001 101.124999) (end 219.264999 101.525001) (width 0.4) (layer F.Cu) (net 5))
 (segment (start 222.205001 101.124999) (end 219.665001 101.124999) (width 0.4) (layer F.Cu) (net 5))
 (segment (start 223.495 99.835) (end 222.205001 101.124999) (width 0.4) (layer F.Cu) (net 5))
 (segment (start 214.184999 100.684999) (end 213.335 99.835) (width 0.4) (layer F.Cu) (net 5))
 (segment (start 214.624999 101.124999) (end 214.184999 100.684999) (width 0.4) (layer F.Cu) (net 5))
 (segment (start 217.164999 101.124999) (end 214.624999 101.124999) (width 0.4) (layer F.Cu) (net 5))
 (segment (start 218.415 102.375) (end 217.164999 101.124999) (width 0.4) (layer F.Cu) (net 5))
 (segment (start 222.86 106.185) (end 219.685 106.185) (width 0.4) (layer F.Cu) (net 5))
 (segment (start 218.415 104.915) (end 218.415 102.375) (width 0.4) (layer F.Cu) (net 5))
 (segment (start 219.685 106.185) (end 218.415 104.915) (width 0.4) (layer F.Cu) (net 5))
 (segment (start 224.13 119.52) (end 224.13 107.455) (width 0.4) (layer F.Cu) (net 5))
 (segment (start 224.13 107.455) (end 222.86 106.185) (width 0.4) (layer F.Cu) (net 5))
 (segment (start 213.335 99.835) (end 213.335 97.93) (width 0.4) (layer F.Cu) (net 5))
 (segment (start 213.335 97.93) (end 212.7 97.295) (width 0.4) (layer F.Cu) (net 5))
 (segment (start 212.7 97.295) (end 205.715 97.295) (width 0.4) (layer F.Cu) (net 5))
 (segment (start 205.08 97.93) (end 205.08 109.606075) (width 0.4) (layer F.Cu) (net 5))
 (segment (start 205.715 97.295) (end 205.08 97.93) (width 0.4) (layer F.Cu) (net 5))
 (segment (start 205.08 109.606075) (end 205.306505 125.461505) (width 0.4) (layer F.Cu) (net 5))
 (segment (start 206.945 127.1) (end 208.89 127.1) (width 0.4) (layer F.Cu) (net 5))
 (segment (start 205.306505 125.461505) (end 206.945 127.1) (width 0.4) (layer F.Cu) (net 5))
 (segment (start 253.34 122.695) (end 253.975 122.06) (width 0.4) (layer F.Cu) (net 7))
 (segment (start 228.175 122.695) (end 253.34 122.695) (width 0.4) (layer F.Cu) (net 7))
 (segment (start 253.975 122.06) (end 253.975 102.375) (width 0.4) (layer F.Cu) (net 7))
 (segment (start 224.13 127.14) (end 224.13 126.74) (width 0.4) (layer F.Cu) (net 7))
 (segment (start 224.13 126.74) (end 228.175 122.695) (width 0.4) (layer F.Cu) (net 7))
 (segment (start 210.795 102.375) (end 210.795 108.09) (width 0.4) (layer F.Cu) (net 3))
 (segment (start 210.795 108.09) (end 216.51 113.805) (width 0.4) (layer F.Cu) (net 3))
 (segment (start 216.51 113.805) (end 216.51 119.52) (width 0.4) (layer F.Cu) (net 3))
 (segment (start 219.05 119.52) (end 219.05 113.17) (width 0.4) (layer F.Cu) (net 4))
 (segment (start 219.05 113.17) (end 213.335 107.455) (width 0.4) (layer F.Cu) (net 4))
 (segment (start 213.335 107.455) (end 213.335 102.375) (width 0.4) (layer F.Cu) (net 4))
 (segment (start 253.34 97.93) (end 251.435 99.835) (width 0.4) (layer F.Cu) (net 6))
 (segment (start 257.15 97.93) (end 253.34 97.93) (width 0.4) (layer F.Cu) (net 6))
 (segment (start 258.42 99.2) (end 257.15 97.93) (width 0.4) (layer F.Cu) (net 6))
 (segment (start 226.67 126.74) (end 228.81 124.6) (width 0.4) (layer F.Cu) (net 6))
 (segment (start 226.67 127.14) (end 226.67 126.74) (width 0.4) (layer F.Cu) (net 6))
 (segment (start 258.42 122.06) (end 258.42 99.2) (width 0.4) (layer F.Cu) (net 6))
 (segment (start 228.81 124.6) (end 255.88 124.6) (width 0.4) (layer F.Cu) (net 6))
 (segment (start 255.88 124.6) (end 258.42 122.06) (width 0.4) (layer F.Cu) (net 6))
 (segment (start 241.91 110.915) (end 241.625 110.63) (width 0.4) (layer F.Cu) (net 17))
 (segment (start 241.91 119.52) (end 241.91 110.915) (width 0.4) (layer F.Cu) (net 17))
 (segment (start 243.625 110.63) (end 243.625 114.25) (width 0.4) (layer F.Cu) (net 18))
 (segment (start 243.625 114.25) (end 244.45 115.075) (width 0.4) (layer F.Cu) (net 18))
 (segment (start 244.45 115.075) (end 244.45 119.52) (width 0.4) (layer F.Cu) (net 18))
 (segment (start 245.625 110.63) (end 245.625 113.075) (width 0.4) (layer F.Cu) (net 19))
 (segment (start 246.99 114.44) (end 246.99 119.52) (width 0.4) (layer F.Cu) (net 19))
 (segment (start 245.625 113.075) (end 246.99 114.44) (width 0.4) (layer F.Cu) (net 19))
 (segment (start 228.925 110.63) (end 228.925 113.52) (width 0.4) (layer F.Cu) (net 14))
 (segment (start 228.925 113.52) (end 232.385 116.98) (width 0.4) (layer F.Cu) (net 14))
 (segment (start 232.385 116.98) (end 233.655 116.98) (width 0.4) (layer F.Cu) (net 14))
 (segment (start 233.655 116.98) (end 234.29 117.615) (width 0.4) (layer F.Cu) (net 14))
 (segment (start 234.29 117.615) (end 234.29 119.52) (width 0.4) (layer F.Cu) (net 14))
 (segment (start 230.925 110.63) (end 230.925 112.98) (width 0.4) (layer F.Cu) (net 15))
 (segment (start 230.925 112.98) (end 233.655 115.71) (width 0.4) (layer F.Cu) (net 15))
 (segment (start 233.655 115.71) (end 236.195 115.71) (width 0.4) (layer F.Cu) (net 15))
 (segment (start 236.83 116.345) (end 236.83 119.52) (width 0.4) (layer F.Cu) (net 15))
 (segment (start 236.195 115.71) (end 236.83 116.345) (width 0.4) (layer F.Cu) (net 15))
 (segment (start 232.925 110.63) (end 232.925 112.44) (width 0.4) (layer F.Cu) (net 16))
 (segment (start 232.925 112.44) (end 234.925 114.44) (width 0.4) (layer F.Cu) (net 16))
 (segment (start 234.925 114.44) (end 238.1 114.44) (width 0.4) (layer F.Cu) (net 16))
 (segment (start 239.37 115.71) (end 239.37 119.52) (width 0.4) (layer F.Cu) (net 16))
 (segment (start 238.1 114.44) (end 239.37 115.71) (width 0.4) (layer F.Cu) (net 16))
 (segment (start 227.4 134.76) (end 231.115 134.76) (width 0.4) (layer F.Cu) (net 11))
 (segment (start 234.29 131.585) (end 234.29 127.14) (width 0.4) (layer F.Cu) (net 11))
 (segment (start 231.115 134.76) (end 234.29 131.585) (width 0.4) (layer F.Cu) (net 11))
 (segment (start 225.4 134.76) (end 225.4 132.855) (width 0.4) (layer F.Cu) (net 12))
 (segment (start 225.4 132.855) (end 226.035 132.22) (width 0.4) (layer F.Cu) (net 12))
 (segment (start 226.035 132.22) (end 230.48 132.22) (width 0.4) (layer F.Cu) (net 12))
 (segment (start 230.48 132.22) (end 231.75 130.95) (width 0.4) (layer F.Cu) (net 12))
 (segment (start 231.75 130.95) (end 231.75 127.14) (width 0.4) (layer F.Cu) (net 12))
 (segment (start 223.4 130.41) (end 223.4 134.76) (width 0.4) (layer F.Cu) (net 13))
 (segment (start 224.13 129.68) (end 223.4 130.41) (width 0.4) (layer F.Cu) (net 13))
 (segment (start 228.27 129.68) (end 224.13 129.68) (width 0.4) (layer F.Cu) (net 13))
 (segment (start 229.21 127.14) (end 229.21 128.74) (width 0.4) (layer F.Cu) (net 13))
 (segment (start 229.21 128.74) (end 228.27 129.68) (width 0.4) (layer F.Cu) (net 13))
 (segment (start 241.56 127.49) (end 241.91 127.14) (width 0.4) (layer F.Cu) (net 8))
 (segment (start 241.56 134.76) (end 241.56 127.49) (width 0.4) (layer F.Cu) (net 8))
 (segment (start 239.37 134.57) (end 239.56 134.76) (width 0.4) (layer F.Cu) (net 9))
 (segment (start 239.37 127.14) (end 239.37 134.57) (width 0.4) (layer F.Cu) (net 9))
 (segment (start 237.56 134.76) (end 237.56 131.68) (width 0.4) (layer F.Cu) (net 10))
 (segment (start 237.56 131.68) (end 236.83 130.95) (width 0.4) (layer F.Cu) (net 10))
 (segment (start 236.83 130.95) (end 236.83 127.14) (width 0.4) (layer F.Cu) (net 10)))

